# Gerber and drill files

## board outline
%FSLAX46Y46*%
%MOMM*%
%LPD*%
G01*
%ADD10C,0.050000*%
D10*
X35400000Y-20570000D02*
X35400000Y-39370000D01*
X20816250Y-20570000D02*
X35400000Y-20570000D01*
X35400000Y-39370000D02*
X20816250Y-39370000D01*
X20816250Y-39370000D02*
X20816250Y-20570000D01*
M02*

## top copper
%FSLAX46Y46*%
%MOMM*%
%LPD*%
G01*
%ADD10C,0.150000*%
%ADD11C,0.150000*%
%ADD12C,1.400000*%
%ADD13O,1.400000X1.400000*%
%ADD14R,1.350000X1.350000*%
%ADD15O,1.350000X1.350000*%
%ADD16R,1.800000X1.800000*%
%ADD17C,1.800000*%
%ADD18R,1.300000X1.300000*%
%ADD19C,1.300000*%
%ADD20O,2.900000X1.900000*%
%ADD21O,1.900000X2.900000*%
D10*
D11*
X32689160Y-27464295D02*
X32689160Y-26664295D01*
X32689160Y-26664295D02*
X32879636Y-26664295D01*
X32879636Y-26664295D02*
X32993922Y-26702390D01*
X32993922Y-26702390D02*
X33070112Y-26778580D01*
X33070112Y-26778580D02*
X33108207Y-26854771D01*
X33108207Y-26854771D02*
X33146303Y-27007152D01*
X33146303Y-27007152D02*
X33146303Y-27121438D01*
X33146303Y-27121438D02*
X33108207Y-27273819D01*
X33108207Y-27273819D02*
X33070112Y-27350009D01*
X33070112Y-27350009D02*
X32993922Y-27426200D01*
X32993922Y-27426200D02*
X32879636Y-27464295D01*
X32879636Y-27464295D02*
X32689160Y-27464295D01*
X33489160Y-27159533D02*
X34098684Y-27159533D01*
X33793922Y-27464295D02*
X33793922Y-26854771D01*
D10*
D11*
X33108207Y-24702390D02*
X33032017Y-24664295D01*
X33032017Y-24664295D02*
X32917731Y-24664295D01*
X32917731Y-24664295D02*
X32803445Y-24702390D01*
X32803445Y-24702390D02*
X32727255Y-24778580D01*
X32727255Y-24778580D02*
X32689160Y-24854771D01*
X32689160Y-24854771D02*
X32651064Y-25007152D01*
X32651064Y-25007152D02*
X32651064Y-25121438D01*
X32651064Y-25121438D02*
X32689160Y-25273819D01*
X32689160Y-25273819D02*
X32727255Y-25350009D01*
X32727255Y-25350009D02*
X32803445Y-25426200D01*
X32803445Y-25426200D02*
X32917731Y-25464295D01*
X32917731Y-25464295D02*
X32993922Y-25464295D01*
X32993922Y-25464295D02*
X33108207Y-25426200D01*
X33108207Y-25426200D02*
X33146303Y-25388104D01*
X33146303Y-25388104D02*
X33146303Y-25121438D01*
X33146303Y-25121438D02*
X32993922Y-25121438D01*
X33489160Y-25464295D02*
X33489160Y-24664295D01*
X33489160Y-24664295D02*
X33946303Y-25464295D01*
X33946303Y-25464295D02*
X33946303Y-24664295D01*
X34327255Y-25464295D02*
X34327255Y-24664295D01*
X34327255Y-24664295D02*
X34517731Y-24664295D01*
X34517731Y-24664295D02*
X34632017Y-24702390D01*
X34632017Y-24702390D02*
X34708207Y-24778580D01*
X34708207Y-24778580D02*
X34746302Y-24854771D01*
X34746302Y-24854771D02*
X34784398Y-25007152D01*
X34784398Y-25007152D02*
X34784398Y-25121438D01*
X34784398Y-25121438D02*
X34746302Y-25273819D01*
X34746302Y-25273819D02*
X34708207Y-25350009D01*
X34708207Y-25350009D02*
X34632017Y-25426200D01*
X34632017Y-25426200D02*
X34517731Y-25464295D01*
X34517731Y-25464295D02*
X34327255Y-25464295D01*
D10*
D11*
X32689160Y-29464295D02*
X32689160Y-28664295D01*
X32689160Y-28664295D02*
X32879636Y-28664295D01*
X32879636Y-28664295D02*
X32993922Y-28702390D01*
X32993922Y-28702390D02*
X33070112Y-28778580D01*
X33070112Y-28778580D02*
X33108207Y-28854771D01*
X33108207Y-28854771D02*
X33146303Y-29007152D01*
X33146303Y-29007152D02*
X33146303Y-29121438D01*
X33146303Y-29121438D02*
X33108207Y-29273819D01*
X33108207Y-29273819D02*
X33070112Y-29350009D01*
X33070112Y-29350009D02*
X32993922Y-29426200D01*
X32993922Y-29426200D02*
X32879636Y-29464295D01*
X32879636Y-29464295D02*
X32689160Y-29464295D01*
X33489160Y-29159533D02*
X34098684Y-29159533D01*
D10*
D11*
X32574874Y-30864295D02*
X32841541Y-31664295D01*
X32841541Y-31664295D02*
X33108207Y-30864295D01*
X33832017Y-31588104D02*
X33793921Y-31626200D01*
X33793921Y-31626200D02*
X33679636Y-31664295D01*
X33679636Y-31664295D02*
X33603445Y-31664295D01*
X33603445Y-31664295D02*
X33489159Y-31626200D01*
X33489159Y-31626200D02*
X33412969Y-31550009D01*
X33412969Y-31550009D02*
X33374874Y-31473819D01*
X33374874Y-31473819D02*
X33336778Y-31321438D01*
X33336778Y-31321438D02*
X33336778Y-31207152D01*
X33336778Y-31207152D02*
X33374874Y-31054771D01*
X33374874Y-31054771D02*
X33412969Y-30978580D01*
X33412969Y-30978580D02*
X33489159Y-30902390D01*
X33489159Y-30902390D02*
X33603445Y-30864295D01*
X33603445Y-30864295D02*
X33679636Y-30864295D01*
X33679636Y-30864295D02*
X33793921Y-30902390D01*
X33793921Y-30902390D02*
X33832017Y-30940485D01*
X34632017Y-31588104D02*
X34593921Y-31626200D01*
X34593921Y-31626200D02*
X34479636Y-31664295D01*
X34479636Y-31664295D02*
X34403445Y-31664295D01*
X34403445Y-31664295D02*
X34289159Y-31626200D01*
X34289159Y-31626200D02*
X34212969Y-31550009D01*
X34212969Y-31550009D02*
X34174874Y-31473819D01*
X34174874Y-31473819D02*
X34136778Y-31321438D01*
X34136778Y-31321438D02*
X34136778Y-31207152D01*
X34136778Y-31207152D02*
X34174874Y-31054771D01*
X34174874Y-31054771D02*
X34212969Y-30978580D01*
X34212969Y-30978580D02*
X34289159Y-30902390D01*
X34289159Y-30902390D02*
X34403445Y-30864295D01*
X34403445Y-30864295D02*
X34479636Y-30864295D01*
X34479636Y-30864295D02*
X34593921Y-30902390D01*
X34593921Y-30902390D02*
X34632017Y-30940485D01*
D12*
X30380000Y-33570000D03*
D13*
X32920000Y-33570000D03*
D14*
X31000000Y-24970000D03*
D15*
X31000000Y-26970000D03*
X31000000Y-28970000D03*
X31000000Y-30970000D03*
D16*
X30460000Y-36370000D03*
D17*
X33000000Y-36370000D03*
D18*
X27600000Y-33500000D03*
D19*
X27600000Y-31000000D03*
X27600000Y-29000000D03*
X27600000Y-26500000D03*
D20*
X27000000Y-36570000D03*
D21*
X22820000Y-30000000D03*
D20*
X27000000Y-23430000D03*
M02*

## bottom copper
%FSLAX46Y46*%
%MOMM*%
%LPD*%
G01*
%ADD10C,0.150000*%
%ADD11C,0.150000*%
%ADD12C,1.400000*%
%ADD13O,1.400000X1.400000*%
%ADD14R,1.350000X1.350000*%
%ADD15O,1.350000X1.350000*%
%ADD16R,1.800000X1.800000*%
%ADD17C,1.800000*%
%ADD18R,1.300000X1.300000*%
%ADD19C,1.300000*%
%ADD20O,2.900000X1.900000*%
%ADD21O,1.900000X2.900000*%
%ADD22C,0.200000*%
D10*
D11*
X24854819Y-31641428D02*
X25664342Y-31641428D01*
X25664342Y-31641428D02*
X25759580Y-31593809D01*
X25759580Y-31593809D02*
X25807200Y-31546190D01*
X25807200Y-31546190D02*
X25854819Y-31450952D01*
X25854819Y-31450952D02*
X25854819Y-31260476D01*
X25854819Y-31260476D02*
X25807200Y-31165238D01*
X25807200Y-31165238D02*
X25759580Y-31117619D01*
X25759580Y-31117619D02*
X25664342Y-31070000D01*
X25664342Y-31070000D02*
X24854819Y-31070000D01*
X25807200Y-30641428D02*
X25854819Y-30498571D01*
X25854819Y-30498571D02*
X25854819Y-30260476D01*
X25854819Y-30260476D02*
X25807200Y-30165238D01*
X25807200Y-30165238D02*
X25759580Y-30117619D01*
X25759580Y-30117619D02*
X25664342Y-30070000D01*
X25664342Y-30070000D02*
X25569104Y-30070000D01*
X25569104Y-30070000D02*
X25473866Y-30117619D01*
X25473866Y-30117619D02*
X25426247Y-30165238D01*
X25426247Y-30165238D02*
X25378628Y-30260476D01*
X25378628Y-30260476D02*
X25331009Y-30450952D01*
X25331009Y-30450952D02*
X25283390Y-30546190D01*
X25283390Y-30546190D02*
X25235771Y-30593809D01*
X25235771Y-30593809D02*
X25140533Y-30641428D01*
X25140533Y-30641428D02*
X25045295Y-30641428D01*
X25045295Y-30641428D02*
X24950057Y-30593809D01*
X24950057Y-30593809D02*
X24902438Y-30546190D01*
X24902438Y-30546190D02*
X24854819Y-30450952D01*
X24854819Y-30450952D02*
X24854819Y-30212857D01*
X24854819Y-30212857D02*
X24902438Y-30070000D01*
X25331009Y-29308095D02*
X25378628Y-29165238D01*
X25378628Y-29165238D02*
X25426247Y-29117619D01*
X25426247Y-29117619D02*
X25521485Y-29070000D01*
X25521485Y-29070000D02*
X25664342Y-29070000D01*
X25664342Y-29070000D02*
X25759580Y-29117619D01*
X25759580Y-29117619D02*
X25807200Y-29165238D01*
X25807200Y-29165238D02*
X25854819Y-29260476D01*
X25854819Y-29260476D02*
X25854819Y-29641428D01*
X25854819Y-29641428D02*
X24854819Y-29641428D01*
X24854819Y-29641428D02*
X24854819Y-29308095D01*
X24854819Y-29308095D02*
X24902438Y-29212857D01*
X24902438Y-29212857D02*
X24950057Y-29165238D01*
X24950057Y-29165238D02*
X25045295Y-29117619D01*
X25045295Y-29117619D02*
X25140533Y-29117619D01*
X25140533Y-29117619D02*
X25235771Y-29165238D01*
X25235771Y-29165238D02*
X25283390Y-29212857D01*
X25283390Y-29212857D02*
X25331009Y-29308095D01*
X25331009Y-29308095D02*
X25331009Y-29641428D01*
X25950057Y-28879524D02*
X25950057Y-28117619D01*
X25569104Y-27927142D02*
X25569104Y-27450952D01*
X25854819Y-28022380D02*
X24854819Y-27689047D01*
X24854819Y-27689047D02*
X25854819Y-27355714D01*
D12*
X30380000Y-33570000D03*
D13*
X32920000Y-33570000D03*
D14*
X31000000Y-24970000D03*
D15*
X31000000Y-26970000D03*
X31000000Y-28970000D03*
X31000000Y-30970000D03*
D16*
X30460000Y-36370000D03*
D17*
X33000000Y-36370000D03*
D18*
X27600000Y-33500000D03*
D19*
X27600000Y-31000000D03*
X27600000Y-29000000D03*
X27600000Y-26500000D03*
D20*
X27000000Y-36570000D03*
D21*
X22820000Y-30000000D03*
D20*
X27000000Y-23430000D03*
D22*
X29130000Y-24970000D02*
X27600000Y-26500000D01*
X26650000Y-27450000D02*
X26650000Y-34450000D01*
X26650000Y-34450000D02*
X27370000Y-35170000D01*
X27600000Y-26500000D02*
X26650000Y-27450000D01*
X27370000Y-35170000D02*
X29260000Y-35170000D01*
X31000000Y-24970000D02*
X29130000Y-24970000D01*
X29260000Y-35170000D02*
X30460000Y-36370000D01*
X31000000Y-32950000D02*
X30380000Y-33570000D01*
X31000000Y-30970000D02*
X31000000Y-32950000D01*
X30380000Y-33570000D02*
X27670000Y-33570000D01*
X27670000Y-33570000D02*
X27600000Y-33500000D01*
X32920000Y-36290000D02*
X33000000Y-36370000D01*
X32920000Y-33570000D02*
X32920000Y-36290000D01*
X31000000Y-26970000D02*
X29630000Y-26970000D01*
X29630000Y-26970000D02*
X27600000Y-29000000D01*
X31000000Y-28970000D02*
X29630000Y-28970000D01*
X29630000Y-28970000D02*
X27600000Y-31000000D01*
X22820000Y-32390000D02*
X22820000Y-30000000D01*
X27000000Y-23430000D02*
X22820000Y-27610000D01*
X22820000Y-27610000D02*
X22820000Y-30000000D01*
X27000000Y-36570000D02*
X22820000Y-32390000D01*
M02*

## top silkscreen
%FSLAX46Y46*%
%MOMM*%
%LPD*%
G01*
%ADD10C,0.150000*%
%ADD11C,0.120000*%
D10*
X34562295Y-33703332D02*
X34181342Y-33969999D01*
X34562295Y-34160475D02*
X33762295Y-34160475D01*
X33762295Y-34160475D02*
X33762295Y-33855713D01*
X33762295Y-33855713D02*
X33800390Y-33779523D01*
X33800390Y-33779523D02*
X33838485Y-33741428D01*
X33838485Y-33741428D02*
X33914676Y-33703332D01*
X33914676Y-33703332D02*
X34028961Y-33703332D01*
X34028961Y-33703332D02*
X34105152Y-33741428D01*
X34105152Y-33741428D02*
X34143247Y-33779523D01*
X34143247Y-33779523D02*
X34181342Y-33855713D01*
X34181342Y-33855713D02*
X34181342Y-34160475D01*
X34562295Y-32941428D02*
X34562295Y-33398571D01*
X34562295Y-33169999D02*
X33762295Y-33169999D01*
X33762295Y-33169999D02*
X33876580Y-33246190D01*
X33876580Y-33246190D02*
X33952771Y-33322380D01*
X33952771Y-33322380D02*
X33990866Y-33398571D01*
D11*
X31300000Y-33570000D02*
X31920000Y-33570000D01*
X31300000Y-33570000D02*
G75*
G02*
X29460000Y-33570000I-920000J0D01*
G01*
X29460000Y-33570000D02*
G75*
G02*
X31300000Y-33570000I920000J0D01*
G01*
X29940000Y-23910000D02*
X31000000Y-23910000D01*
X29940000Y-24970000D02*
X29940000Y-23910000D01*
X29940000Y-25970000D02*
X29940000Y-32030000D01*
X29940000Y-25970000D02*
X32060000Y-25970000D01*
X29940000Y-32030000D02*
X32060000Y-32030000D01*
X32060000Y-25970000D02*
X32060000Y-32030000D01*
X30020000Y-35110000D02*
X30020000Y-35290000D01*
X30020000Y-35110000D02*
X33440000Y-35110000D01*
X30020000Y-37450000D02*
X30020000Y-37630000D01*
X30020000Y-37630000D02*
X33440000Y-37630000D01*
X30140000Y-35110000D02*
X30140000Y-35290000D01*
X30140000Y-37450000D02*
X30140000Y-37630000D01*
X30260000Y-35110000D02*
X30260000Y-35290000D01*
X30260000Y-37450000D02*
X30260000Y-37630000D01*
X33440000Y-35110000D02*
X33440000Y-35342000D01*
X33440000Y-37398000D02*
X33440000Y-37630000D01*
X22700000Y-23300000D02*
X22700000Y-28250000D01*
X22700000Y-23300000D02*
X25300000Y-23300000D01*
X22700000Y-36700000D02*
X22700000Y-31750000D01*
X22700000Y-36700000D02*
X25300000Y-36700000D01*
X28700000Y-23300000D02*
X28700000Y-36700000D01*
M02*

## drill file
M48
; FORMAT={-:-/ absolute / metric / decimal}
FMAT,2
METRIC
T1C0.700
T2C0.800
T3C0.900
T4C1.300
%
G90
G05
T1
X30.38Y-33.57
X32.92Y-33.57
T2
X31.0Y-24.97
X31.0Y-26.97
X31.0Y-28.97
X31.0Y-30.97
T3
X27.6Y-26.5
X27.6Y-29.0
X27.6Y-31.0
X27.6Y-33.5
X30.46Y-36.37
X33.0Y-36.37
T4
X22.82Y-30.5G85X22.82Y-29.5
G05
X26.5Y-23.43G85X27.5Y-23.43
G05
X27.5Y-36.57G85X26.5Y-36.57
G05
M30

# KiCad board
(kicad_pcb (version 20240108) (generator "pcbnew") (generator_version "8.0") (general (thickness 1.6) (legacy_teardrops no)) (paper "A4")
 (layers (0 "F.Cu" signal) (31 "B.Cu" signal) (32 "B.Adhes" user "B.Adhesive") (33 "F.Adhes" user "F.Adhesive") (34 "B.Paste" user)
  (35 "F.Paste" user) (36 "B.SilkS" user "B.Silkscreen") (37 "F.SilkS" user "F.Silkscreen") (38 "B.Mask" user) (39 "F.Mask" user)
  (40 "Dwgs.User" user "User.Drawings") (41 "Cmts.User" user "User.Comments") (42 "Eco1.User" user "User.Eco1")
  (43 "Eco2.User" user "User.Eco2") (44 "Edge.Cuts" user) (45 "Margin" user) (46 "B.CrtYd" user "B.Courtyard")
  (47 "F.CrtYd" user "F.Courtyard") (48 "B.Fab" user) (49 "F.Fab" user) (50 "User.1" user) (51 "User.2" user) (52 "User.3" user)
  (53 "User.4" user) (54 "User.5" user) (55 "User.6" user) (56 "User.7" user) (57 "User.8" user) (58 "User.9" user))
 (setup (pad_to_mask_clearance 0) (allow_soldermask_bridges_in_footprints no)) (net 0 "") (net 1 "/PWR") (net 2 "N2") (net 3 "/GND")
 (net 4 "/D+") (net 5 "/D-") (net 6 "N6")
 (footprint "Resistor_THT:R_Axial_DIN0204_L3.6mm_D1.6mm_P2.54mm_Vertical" (layer "F.Cu") (at 30.38 33.57)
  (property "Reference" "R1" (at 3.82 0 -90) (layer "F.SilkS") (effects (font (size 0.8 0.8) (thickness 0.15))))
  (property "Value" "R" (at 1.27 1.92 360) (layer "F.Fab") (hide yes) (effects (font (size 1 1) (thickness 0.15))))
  (fp_line (start 0.92 0) (end 1.54 0) (stroke (width 0.12) (type solid)) (layer "F.SilkS"))
  (fp_circle (center 0 0) (end 0.92 0) (stroke (width 0.12) (type solid)) (fill none) (layer "F.SilkS"))
  (pad "1" thru_hole circle (at 0 0) (size 1.4 1.4) (drill 0.7) (layers "*.Cu" "*.Mask") (remove_unused_layers no) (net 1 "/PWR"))
  (pad "2" thru_hole oval (at 2.54 0) (size 1.4 1.4) (drill 0.7) (layers "*.Cu" "*.Mask") (remove_unused_layers no) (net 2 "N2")))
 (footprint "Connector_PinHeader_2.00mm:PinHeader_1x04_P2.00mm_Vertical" (layer "F.Cu") (at 31 24.97)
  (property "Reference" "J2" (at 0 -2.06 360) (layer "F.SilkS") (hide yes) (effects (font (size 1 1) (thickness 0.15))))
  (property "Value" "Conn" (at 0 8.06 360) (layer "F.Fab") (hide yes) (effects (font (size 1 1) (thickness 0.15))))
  (fp_line (start -1.06 -1.06) (end 0 -1.06) (stroke (width 0.12) (type solid)) (layer "F.SilkS"))
  (fp_line (start -1.06 0) (end -1.06 -1.06) (stroke (width 0.12) (type solid)) (layer "F.SilkS"))
  (fp_line (start -1.06 1) (end -1.06 7.06) (stroke (width 0.12) (type solid)) (layer "F.SilkS"))
  (fp_line (start -1.06 1) (end 1.06 1) (stroke (width 0.12) (type solid)) (layer "F.SilkS"))
  (fp_line (start -1.06 7.06) (end 1.06 7.06) (stroke (width 0.12) (type solid)) (layer "F.SilkS"))
  (fp_line (start 1.06 1) (end 1.06 7.06) (stroke (width 0.12) (type solid)) (layer "F.SilkS"))
  (pad "1" thru_hole rect (at 0 0) (size 1.35 1.35) (drill 0.8) (layers "*.Cu" "*.Mask") (remove_unused_layers no) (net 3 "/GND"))
  (pad "2" thru_hole oval (at 0 2) (size 1.35 1.35) (drill 0.8) (layers "*.Cu" "*.Mask") (remove_unused_layers no) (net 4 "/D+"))
  (pad "3" thru_hole oval (at 0 4) (size 1.35 1.35) (drill 0.8) (layers "*.Cu" "*.Mask") (remove_unused_layers no) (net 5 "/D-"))
  (pad "4" thru_hole oval (at 0 6) (size 1.35 1.35) (drill 0.8) (layers "*.Cu" "*.Mask") (remove_unused_layers no) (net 1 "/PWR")))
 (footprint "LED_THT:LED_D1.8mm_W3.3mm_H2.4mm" (layer "F.Cu") (at 30.46 36.37)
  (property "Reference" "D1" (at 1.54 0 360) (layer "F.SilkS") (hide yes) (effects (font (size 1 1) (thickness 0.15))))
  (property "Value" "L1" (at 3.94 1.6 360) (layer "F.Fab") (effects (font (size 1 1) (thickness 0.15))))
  (fp_line (start -0.44 -1.26) (end -0.44 -1.08) (stroke (width 0.12) (type solid)) (layer "F.SilkS"))
  (fp_line (start -0.44 -1.26) (end 2.98 -1.26) (stroke (width 0.12) (type solid)) (layer "F.SilkS"))
  (fp_line (start -0.44 1.08) (end -0.44 1.26) (stroke (width 0.12) (type solid)) (layer "F.SilkS"))
  (fp_line (start -0.44 1.26) (end 2.98 1.26) (stroke (width 0.12) (type solid)) (layer "F.SilkS"))
  (fp_line (start -0.32 -1.26) (end -0.32 -1.08) (stroke (width 0.12) (type solid)) (layer "F.SilkS"))
  (fp_line (start -0.32 1.08) (end -0.32 1.26) (stroke (width 0.12) (type solid)) (layer "F.SilkS"))
  (fp_line (start -0.2 -1.26) (end -0.2 -1.08) (stroke (width 0.12) (type solid)) (layer "F.SilkS"))
  (fp_line (start -0.2 1.08) (end -0.2 1.26) (stroke (width 0.12) (type solid)) (layer "F.SilkS"))
  (fp_line (start 2.98 -1.26) (end 2.98 -1.028) (stroke (width 0.12) (type solid)) (layer "F.SilkS"))
  (fp_line (start 2.98 1.028) (end 2.98 1.26) (stroke (width 0.12) (type solid)) (layer "F.SilkS"))
  (pad "1" thru_hole rect (at 0 0) (size 1.8 1.8) (drill 0.9) (layers "*.Cu" "*.Mask") (remove_unused_layers no) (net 3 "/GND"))
  (pad "2" thru_hole circle (at 2.54 0) (size 1.8 1.8) (drill 0.9) (layers "*.Cu" "*.Mask") (remove_unused_layers no) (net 2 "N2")))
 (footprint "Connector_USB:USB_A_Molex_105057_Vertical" (layer "F.Cu") (at 27.6 33.5 90)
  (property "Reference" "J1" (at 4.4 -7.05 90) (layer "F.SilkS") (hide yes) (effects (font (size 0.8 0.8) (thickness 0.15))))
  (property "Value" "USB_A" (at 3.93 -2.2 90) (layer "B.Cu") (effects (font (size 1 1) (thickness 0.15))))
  (fp_line (start 10.2 -4.9) (end 5.25 -4.9) (stroke (width 0.12) (type solid)) (layer "F.SilkS"))
  (fp_line (start 10.2 -4.9) (end 10.2 -2.3) (stroke (width 0.12) (type solid)) (layer "F.SilkS"))
  (fp_line (start -3.2 -4.9) (end 1.75 -4.9) (stroke (width 0.12) (type solid)) (layer "F.SilkS"))
  (fp_line (start -3.2 -4.9) (end -3.2 -2.3) (stroke (width 0.12) (type solid)) (layer "F.SilkS"))
  (fp_line (start 10.2 1.1) (end -3.2 1.1) (stroke (width 0.12) (type solid)) (layer "F.SilkS"))
  (pad "1" thru_hole rect (at 0 0 90) (size 1.3 1.3) (drill 0.9) (layers "*.Cu" "*.Mask") (remove_unused_layers no) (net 1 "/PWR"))
  (pad "2" thru_hole circle (at 2.5 0 90) (size 1.3 1.3) (drill 0.9) (layers "*.Cu" "*.Mask") (remove_unused_layers no) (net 5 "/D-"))
  (pad "3" thru_hole circle (at 4.5 0 90) (size 1.3 1.3) (drill 0.9) (layers "*.Cu" "*.Mask") (remove_unused_layers no) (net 4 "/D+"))
  (pad "4" thru_hole circle (at 7 0 90) (size 1.3 1.3) (drill 0.9) (layers "*.Cu" "*.Mask") (remove_unused_layers no) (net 3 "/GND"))
  (pad "5" thru_hole oval (at -3.07 -0.6 270) (size 1.9 2.9) (drill oval 1.3 2.3) (layers "*.Cu" "*.Mask") (remove_unused_layers no)
   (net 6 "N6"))
  (pad "5" thru_hole oval (at 3.5 -4.78 180) (size 1.9 2.9) (drill oval 1.3 2.3) (layers "*.Cu" "*.Mask") (remove_unused_layers no)
   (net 6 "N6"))
  (pad "5" thru_hole oval (at 10.07 -0.6 90) (size 1.9 2.9) (drill oval 1.3 2.3) (layers "*.Cu" "*.Mask") (remove_unused_layers no)
   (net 6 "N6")))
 (gr_line (start 35.4 20.57) (end 35.4 39.37) (stroke (width 0.05) (type default)) (layer "Edge.Cuts"))
 (gr_line (start 20.81625 20.57) (end 35.4 20.57) (stroke (width 0.05) (type default)) (layer "Edge.Cuts"))
 (gr_line (start 35.4 39.37) (end 20.81625 39.37) (stroke (width 0.05) (type default)) (layer "Edge.Cuts"))
 (gr_line (start 20.81625 39.37) (end 20.81625 20.57) (stroke (width 0.05) (type default)) (layer "Edge.Cuts"))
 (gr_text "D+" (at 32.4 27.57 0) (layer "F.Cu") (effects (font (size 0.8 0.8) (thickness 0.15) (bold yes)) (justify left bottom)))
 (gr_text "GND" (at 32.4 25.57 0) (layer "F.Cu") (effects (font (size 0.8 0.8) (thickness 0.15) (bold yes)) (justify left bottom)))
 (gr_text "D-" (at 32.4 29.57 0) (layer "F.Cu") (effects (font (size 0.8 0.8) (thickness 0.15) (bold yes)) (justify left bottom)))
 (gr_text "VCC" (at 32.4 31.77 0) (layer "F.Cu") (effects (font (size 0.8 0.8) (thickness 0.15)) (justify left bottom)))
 (segment (start 29.13 24.97) (end 27.6 26.5) (width 0.2) (layer "B.Cu") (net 3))
 (segment (start 26.65 27.45) (end 26.65 34.45) (width 0.2) (layer "B.Cu") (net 3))
 (segment (start 26.65 34.45) (end 27.37 35.17) (width 0.2) (layer "B.Cu") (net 3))
 (segment (start 27.6 26.5) (end 26.65 27.45) (width 0.2) (layer "B.Cu") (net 3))
 (segment (start 27.37 35.17) (end 29.26 35.17) (width 0.2) (layer "B.Cu") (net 3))
 (segment (start 31 24.97) (end 29.13 24.97) (width 0.2) (layer "B.Cu") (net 3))
 (segment (start 29.26 35.17) (end 30.46 36.37) (width 0.2) (layer "B.Cu") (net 3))
 (segment (start 31 32.95) (end 30.38 33.57) (width 0.2) (layer "B.Cu") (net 1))
 (segment (start 31 30.97) (end 31 32.95) (width 0.2) (layer "B.Cu") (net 1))
 (segment (start 30.38 33.57) (end 27.67 33.57) (width 0.2) (layer "B.Cu") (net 1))
 (segment (start 27.67 33.57) (end 27.6 33.5) (width 0.2) (layer "B.Cu") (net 1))
 (segment (start 32.92 36.29) (end 33 36.37) (width 0.2) (layer "B.Cu") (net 2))
 (segment (start 32.92 33.57) (end 32.92 36.29) (width 0.2) (layer "B.Cu") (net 2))
 (segment (start 31 26.97) (end 29.63 26.97) (width 0.2) (layer "B.Cu") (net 4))
 (segment (start 29.63 26.97) (end 27.6 29) (width 0.2) (layer "B.Cu") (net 4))
 (segment (start 31 28.97) (end 29.63 28.97) (width 0.2) (layer "B.Cu") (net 5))
 (segment (start 29.63 28.97) (end 27.6 31) (width 0.2) (layer "B.Cu") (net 5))
 (segment (start 22.82 32.39) (end 22.82 30) (width 0.2) (layer "B.Cu") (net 6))
 (segment (start 27 23.43) (end 22.82 27.61) (width 0.2) (layer "B.Cu") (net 6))
 (segment (start 22.82 27.61) (end 22.82 30) (width 0.2) (layer "B.Cu") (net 6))
 (segment (start 27 36.57) (end 22.82 32.39) (width 0.2) (layer "B.Cu") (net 6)))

